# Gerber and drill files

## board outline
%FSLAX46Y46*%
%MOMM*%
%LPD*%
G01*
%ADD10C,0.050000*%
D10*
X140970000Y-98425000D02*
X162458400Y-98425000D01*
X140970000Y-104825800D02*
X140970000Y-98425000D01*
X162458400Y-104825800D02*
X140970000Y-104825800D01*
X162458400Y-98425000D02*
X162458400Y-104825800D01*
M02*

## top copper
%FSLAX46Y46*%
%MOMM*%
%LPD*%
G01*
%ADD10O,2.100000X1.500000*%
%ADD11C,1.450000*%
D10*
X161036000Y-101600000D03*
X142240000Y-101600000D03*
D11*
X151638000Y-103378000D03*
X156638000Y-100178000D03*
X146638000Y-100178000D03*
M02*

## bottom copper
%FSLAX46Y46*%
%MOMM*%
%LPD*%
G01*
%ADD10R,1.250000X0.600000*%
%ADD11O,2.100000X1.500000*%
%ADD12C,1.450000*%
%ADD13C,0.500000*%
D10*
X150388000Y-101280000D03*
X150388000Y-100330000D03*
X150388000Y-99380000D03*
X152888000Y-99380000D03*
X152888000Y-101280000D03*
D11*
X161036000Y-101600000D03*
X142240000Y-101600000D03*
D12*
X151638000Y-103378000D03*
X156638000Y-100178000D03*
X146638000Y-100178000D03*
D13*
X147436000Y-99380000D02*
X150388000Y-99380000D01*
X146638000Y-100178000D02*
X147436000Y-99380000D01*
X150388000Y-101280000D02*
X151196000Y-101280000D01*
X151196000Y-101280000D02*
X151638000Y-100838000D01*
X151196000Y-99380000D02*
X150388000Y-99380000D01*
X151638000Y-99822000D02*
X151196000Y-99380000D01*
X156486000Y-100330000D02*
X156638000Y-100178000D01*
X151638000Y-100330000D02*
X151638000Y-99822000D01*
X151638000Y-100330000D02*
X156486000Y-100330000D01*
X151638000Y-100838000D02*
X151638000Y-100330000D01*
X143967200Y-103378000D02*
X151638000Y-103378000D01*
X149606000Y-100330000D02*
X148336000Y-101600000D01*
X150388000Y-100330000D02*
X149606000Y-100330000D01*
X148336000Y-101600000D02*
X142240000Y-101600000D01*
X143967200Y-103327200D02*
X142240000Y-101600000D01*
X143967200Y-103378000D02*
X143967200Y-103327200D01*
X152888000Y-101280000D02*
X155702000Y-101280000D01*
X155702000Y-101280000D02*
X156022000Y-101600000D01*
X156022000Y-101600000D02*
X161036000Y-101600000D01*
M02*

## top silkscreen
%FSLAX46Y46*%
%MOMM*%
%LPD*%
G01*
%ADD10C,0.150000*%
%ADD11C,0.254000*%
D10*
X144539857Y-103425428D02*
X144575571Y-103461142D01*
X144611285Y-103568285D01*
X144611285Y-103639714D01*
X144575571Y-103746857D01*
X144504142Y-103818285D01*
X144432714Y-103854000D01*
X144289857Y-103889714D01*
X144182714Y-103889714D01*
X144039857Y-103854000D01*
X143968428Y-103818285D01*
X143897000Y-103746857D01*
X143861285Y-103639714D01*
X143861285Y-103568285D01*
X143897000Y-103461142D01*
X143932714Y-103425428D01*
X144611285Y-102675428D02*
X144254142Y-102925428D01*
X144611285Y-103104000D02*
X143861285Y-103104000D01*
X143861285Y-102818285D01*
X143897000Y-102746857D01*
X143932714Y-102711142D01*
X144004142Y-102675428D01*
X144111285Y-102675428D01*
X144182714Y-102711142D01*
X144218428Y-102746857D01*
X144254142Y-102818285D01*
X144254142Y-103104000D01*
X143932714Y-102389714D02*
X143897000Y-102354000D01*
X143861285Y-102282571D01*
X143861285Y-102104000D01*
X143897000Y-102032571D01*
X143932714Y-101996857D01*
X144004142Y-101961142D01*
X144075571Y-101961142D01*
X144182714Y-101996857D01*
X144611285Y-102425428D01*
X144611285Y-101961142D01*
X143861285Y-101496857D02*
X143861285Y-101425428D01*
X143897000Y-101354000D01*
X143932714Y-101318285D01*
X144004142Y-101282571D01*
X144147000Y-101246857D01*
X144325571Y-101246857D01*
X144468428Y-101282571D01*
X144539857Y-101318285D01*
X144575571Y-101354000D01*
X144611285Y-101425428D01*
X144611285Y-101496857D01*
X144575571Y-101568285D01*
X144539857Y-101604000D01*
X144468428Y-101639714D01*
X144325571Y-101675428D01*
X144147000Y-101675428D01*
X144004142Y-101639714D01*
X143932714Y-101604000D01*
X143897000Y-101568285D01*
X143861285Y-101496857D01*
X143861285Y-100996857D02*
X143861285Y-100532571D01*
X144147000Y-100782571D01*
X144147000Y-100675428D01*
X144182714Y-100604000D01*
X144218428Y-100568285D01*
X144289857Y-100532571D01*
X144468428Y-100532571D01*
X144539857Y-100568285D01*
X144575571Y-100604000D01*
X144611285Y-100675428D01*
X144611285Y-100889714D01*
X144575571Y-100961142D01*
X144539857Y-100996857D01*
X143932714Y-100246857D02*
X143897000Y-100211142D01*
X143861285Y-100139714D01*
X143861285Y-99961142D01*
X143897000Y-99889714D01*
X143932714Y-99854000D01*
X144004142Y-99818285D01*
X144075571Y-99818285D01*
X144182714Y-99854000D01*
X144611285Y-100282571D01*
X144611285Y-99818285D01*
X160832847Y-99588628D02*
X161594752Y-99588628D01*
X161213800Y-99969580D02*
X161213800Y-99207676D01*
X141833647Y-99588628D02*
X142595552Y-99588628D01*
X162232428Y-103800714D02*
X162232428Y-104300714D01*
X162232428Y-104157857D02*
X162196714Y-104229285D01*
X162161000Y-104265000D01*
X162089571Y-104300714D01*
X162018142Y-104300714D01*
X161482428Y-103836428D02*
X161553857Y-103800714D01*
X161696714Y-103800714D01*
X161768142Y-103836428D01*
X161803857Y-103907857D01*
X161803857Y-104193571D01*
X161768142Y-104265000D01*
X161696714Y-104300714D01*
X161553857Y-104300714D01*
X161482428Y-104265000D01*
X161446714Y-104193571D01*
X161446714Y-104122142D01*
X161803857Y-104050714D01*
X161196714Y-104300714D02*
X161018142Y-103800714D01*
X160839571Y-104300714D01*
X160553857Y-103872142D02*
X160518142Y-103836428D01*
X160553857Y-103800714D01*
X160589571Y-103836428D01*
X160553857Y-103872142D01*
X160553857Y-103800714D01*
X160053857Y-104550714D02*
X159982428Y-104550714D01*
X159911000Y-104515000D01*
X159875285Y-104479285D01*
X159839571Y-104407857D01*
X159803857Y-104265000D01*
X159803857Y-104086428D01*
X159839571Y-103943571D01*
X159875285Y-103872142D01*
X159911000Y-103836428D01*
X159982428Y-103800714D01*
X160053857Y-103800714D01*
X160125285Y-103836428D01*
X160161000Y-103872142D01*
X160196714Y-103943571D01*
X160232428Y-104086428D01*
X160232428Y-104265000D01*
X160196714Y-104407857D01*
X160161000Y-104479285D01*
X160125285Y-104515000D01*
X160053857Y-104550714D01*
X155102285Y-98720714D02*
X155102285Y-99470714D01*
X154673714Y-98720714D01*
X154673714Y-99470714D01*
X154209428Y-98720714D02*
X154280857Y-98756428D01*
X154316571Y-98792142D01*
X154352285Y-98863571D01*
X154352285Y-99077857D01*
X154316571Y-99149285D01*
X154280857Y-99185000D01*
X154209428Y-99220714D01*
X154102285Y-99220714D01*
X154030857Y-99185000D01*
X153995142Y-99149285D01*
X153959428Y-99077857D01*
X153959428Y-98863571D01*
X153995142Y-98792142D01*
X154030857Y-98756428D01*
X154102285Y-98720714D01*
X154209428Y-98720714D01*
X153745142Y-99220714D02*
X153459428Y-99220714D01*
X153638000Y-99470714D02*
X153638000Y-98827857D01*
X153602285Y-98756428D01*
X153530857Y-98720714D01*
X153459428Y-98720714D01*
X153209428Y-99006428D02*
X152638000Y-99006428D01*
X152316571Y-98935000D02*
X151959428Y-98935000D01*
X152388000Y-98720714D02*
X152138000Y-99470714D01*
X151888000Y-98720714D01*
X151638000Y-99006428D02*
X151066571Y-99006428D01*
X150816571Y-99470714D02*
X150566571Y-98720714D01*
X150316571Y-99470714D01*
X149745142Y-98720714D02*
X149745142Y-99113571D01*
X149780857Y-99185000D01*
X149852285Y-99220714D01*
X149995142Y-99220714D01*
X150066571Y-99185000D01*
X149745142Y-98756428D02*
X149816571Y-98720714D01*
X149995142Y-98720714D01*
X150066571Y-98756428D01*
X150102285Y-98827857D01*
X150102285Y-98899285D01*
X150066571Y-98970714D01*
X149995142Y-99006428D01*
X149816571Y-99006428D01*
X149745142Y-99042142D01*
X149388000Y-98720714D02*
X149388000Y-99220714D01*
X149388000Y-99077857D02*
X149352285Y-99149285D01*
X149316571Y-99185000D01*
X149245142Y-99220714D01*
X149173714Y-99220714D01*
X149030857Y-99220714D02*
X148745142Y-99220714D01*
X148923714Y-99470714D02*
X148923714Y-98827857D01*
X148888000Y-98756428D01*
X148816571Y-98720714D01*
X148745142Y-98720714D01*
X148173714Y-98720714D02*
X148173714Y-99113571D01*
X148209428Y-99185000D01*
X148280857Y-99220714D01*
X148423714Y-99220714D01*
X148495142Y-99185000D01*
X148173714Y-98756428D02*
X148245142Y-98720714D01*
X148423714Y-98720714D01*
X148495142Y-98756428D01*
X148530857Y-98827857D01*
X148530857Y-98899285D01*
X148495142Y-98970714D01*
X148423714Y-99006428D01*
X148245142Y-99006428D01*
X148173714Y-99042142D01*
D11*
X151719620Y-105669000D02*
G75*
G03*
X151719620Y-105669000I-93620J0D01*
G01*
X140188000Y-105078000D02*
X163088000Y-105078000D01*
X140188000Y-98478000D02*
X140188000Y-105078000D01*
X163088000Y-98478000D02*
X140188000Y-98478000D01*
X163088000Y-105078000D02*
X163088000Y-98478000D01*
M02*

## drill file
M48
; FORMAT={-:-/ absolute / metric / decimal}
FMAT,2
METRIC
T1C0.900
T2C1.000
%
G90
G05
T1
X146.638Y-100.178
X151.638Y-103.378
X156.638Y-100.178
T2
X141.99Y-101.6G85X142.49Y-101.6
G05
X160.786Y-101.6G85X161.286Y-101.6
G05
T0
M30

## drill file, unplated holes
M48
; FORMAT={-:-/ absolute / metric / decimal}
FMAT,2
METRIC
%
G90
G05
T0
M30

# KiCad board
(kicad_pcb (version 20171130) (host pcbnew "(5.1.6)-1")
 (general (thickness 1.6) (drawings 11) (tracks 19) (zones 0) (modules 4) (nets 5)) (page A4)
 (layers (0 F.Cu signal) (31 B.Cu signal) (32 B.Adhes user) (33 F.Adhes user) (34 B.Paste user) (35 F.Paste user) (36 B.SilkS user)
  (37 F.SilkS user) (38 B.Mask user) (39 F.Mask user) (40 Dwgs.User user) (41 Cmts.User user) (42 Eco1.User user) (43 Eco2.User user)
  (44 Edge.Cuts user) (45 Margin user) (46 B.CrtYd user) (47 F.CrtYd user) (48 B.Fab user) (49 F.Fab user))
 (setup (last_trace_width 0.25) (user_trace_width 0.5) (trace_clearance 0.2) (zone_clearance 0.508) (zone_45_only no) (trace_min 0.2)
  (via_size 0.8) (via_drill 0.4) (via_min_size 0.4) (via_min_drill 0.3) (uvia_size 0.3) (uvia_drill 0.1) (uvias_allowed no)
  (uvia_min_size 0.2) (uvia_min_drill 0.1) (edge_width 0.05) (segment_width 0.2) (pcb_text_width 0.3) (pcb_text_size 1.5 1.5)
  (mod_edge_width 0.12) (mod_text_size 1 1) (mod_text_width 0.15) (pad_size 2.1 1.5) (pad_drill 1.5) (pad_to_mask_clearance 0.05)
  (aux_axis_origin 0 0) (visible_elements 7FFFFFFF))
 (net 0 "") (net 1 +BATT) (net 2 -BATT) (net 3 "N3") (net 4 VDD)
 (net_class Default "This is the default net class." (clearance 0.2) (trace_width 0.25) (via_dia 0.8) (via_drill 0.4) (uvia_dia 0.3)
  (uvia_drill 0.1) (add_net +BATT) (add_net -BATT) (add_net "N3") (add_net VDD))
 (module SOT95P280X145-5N (layer B.Cu) (at 151.638 100.33)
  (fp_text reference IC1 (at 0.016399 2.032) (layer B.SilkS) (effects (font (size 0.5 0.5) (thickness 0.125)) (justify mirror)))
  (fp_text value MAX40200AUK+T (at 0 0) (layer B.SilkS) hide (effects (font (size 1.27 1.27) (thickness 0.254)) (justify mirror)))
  (pad 1 smd rect (at -1.25 0.95 270) (size 0.6 1.25) (layers B.Cu B.Paste B.Mask) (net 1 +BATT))
  (pad 2 smd rect (at -1.25 0 270) (size 0.6 1.25) (layers B.Cu B.Paste B.Mask) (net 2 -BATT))
  (pad 3 smd rect (at -1.25 -0.95 270) (size 0.6 1.25) (layers B.Cu B.Paste B.Mask) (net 1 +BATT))
  (pad 4 smd rect (at 1.25 -0.95 270) (size 0.6 1.25) (layers B.Cu B.Paste B.Mask) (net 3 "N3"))
  (pad 5 smd rect (at 1.25 0.95 270) (size 0.6 1.25) (layers B.Cu B.Paste B.Mask) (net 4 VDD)))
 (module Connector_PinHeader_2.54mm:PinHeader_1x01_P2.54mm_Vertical (layer B.Cu) (at 161.036 101.6)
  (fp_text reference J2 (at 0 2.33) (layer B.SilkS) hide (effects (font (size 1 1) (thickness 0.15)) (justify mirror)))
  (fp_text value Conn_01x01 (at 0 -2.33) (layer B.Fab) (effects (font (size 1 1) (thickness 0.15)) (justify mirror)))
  (pad 1 thru_hole oval (at 0 0) (size 2.1 1.5) (drill oval 1.5 1) (layers *.Cu *.Mask) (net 4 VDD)))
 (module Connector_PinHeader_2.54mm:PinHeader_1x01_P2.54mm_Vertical (layer B.Cu) (at 142.24 101.6)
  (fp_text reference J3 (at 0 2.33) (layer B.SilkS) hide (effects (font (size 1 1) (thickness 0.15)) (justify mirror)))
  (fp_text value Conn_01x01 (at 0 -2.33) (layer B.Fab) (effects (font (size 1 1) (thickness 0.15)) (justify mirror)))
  (pad 1 thru_hole oval (at 0 0) (size 2.1 1.5) (drill oval 1.5 1) (layers *.Cu *.Mask) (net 2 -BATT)))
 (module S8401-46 (layer F.Cu) (at 151.638 101.778 180)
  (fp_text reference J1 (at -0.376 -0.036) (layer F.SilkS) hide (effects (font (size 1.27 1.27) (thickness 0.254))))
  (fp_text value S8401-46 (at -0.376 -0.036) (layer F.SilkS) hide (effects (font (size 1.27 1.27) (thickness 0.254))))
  (fp_circle (center 0.012 -3.891) (end 0.012 -3.79738) (layer F.SilkS) (width 0.254))
  (fp_line (start 11.45 -3.3) (end -11.45 -3.3) (layer F.SilkS) (width 0.254))
  (fp_line (start 11.45 3.3) (end 11.45 -3.3) (layer F.SilkS) (width 0.254))
  (fp_line (start -11.45 3.3) (end 11.45 3.3) (layer F.SilkS) (width 0.254))
  (fp_line (start -11.45 -3.3) (end -11.45 3.3) (layer F.SilkS) (width 0.254))
  (pad 1 thru_hole circle (at 0 -1.6 180) (size 1.45 1.45) (drill 0.9) (layers *.Cu *.Mask) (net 2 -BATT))
  (pad 2 thru_hole circle (at -5 1.6 180) (size 1.45 1.45) (drill 0.9) (layers *.Cu *.Mask) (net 1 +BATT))
  (pad 3 thru_hole circle (at 5 1.6 180) (size 1.45 1.45) (drill 0.9) (layers *.Cu *.Mask) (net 1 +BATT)))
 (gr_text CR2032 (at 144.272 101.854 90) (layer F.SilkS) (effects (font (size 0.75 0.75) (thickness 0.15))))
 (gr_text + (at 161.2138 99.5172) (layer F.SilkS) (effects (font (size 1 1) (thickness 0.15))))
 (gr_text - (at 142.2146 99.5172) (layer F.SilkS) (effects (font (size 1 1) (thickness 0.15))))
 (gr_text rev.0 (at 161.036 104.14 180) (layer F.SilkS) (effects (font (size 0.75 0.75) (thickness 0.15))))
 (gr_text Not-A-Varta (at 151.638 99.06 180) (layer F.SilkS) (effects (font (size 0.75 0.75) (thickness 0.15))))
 (gr_line (start 140.97 98.425) (end 162.4584 98.425) (layer Edge.Cuts) (width 0.05))
 (gr_line (start 140.97 104.8258) (end 140.97 98.425) (layer Edge.Cuts) (width 0.05))
 (gr_line (start 162.4584 104.8258) (end 140.97 104.8258) (layer Edge.Cuts) (width 0.05))
 (gr_line (start 162.4584 98.425) (end 162.4584 104.8258) (layer Edge.Cuts) (width 0.05))
 (segment (start 147.436 99.38) (end 150.388 99.38) (width 0.5) (layer B.Cu) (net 1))
 (segment (start 146.638 100.178) (end 147.436 99.38) (width 0.5) (layer B.Cu) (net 1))
 (segment (start 150.388 101.28) (end 151.196 101.28) (width 0.5) (layer B.Cu) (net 1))
 (segment (start 151.196 101.28) (end 151.638 100.838) (width 0.5) (layer B.Cu) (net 1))
 (segment (start 151.196 99.38) (end 150.388 99.38) (width 0.5) (layer B.Cu) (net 1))
 (segment (start 151.638 99.822) (end 151.196 99.38) (width 0.5) (layer B.Cu) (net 1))
 (segment (start 156.486 100.33) (end 156.638 100.178) (width 0.5) (layer B.Cu) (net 1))
 (segment (start 151.638 100.33) (end 151.638 99.822) (width 0.5) (layer B.Cu) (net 1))
 (segment (start 151.638 100.33) (end 156.486 100.33) (width 0.5) (layer B.Cu) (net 1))
 (segment (start 151.638 100.838) (end 151.638 100.33) (width 0.5) (layer B.Cu) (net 1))
 (segment (start 143.9672 103.378) (end 151.638 103.378) (width 0.5) (layer B.Cu) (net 2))
 (segment (start 149.606 100.33) (end 148.336 101.6) (width 0.5) (layer B.Cu) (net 2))
 (segment (start 150.388 100.33) (end 149.606 100.33) (width 0.5) (layer B.Cu) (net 2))
 (segment (start 148.336 101.6) (end 142.24 101.6) (width 0.5) (layer B.Cu) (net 2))
 (segment (start 143.9672 103.3272) (end 142.24 101.6) (width 0.5) (layer B.Cu) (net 2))
 (segment (start 143.9672 103.378) (end 143.9672 103.3272) (width 0.5) (layer B.Cu) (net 2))
 (segment (start 152.888 101.28) (end 155.702 101.28) (width 0.5) (layer B.Cu) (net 4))
 (segment (start 155.702 101.28) (end 156.022 101.6) (width 0.5) (layer B.Cu) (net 4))
 (segment (start 156.022 101.6) (end 161.036 101.6) (width 0.5) (layer B.Cu) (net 4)))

